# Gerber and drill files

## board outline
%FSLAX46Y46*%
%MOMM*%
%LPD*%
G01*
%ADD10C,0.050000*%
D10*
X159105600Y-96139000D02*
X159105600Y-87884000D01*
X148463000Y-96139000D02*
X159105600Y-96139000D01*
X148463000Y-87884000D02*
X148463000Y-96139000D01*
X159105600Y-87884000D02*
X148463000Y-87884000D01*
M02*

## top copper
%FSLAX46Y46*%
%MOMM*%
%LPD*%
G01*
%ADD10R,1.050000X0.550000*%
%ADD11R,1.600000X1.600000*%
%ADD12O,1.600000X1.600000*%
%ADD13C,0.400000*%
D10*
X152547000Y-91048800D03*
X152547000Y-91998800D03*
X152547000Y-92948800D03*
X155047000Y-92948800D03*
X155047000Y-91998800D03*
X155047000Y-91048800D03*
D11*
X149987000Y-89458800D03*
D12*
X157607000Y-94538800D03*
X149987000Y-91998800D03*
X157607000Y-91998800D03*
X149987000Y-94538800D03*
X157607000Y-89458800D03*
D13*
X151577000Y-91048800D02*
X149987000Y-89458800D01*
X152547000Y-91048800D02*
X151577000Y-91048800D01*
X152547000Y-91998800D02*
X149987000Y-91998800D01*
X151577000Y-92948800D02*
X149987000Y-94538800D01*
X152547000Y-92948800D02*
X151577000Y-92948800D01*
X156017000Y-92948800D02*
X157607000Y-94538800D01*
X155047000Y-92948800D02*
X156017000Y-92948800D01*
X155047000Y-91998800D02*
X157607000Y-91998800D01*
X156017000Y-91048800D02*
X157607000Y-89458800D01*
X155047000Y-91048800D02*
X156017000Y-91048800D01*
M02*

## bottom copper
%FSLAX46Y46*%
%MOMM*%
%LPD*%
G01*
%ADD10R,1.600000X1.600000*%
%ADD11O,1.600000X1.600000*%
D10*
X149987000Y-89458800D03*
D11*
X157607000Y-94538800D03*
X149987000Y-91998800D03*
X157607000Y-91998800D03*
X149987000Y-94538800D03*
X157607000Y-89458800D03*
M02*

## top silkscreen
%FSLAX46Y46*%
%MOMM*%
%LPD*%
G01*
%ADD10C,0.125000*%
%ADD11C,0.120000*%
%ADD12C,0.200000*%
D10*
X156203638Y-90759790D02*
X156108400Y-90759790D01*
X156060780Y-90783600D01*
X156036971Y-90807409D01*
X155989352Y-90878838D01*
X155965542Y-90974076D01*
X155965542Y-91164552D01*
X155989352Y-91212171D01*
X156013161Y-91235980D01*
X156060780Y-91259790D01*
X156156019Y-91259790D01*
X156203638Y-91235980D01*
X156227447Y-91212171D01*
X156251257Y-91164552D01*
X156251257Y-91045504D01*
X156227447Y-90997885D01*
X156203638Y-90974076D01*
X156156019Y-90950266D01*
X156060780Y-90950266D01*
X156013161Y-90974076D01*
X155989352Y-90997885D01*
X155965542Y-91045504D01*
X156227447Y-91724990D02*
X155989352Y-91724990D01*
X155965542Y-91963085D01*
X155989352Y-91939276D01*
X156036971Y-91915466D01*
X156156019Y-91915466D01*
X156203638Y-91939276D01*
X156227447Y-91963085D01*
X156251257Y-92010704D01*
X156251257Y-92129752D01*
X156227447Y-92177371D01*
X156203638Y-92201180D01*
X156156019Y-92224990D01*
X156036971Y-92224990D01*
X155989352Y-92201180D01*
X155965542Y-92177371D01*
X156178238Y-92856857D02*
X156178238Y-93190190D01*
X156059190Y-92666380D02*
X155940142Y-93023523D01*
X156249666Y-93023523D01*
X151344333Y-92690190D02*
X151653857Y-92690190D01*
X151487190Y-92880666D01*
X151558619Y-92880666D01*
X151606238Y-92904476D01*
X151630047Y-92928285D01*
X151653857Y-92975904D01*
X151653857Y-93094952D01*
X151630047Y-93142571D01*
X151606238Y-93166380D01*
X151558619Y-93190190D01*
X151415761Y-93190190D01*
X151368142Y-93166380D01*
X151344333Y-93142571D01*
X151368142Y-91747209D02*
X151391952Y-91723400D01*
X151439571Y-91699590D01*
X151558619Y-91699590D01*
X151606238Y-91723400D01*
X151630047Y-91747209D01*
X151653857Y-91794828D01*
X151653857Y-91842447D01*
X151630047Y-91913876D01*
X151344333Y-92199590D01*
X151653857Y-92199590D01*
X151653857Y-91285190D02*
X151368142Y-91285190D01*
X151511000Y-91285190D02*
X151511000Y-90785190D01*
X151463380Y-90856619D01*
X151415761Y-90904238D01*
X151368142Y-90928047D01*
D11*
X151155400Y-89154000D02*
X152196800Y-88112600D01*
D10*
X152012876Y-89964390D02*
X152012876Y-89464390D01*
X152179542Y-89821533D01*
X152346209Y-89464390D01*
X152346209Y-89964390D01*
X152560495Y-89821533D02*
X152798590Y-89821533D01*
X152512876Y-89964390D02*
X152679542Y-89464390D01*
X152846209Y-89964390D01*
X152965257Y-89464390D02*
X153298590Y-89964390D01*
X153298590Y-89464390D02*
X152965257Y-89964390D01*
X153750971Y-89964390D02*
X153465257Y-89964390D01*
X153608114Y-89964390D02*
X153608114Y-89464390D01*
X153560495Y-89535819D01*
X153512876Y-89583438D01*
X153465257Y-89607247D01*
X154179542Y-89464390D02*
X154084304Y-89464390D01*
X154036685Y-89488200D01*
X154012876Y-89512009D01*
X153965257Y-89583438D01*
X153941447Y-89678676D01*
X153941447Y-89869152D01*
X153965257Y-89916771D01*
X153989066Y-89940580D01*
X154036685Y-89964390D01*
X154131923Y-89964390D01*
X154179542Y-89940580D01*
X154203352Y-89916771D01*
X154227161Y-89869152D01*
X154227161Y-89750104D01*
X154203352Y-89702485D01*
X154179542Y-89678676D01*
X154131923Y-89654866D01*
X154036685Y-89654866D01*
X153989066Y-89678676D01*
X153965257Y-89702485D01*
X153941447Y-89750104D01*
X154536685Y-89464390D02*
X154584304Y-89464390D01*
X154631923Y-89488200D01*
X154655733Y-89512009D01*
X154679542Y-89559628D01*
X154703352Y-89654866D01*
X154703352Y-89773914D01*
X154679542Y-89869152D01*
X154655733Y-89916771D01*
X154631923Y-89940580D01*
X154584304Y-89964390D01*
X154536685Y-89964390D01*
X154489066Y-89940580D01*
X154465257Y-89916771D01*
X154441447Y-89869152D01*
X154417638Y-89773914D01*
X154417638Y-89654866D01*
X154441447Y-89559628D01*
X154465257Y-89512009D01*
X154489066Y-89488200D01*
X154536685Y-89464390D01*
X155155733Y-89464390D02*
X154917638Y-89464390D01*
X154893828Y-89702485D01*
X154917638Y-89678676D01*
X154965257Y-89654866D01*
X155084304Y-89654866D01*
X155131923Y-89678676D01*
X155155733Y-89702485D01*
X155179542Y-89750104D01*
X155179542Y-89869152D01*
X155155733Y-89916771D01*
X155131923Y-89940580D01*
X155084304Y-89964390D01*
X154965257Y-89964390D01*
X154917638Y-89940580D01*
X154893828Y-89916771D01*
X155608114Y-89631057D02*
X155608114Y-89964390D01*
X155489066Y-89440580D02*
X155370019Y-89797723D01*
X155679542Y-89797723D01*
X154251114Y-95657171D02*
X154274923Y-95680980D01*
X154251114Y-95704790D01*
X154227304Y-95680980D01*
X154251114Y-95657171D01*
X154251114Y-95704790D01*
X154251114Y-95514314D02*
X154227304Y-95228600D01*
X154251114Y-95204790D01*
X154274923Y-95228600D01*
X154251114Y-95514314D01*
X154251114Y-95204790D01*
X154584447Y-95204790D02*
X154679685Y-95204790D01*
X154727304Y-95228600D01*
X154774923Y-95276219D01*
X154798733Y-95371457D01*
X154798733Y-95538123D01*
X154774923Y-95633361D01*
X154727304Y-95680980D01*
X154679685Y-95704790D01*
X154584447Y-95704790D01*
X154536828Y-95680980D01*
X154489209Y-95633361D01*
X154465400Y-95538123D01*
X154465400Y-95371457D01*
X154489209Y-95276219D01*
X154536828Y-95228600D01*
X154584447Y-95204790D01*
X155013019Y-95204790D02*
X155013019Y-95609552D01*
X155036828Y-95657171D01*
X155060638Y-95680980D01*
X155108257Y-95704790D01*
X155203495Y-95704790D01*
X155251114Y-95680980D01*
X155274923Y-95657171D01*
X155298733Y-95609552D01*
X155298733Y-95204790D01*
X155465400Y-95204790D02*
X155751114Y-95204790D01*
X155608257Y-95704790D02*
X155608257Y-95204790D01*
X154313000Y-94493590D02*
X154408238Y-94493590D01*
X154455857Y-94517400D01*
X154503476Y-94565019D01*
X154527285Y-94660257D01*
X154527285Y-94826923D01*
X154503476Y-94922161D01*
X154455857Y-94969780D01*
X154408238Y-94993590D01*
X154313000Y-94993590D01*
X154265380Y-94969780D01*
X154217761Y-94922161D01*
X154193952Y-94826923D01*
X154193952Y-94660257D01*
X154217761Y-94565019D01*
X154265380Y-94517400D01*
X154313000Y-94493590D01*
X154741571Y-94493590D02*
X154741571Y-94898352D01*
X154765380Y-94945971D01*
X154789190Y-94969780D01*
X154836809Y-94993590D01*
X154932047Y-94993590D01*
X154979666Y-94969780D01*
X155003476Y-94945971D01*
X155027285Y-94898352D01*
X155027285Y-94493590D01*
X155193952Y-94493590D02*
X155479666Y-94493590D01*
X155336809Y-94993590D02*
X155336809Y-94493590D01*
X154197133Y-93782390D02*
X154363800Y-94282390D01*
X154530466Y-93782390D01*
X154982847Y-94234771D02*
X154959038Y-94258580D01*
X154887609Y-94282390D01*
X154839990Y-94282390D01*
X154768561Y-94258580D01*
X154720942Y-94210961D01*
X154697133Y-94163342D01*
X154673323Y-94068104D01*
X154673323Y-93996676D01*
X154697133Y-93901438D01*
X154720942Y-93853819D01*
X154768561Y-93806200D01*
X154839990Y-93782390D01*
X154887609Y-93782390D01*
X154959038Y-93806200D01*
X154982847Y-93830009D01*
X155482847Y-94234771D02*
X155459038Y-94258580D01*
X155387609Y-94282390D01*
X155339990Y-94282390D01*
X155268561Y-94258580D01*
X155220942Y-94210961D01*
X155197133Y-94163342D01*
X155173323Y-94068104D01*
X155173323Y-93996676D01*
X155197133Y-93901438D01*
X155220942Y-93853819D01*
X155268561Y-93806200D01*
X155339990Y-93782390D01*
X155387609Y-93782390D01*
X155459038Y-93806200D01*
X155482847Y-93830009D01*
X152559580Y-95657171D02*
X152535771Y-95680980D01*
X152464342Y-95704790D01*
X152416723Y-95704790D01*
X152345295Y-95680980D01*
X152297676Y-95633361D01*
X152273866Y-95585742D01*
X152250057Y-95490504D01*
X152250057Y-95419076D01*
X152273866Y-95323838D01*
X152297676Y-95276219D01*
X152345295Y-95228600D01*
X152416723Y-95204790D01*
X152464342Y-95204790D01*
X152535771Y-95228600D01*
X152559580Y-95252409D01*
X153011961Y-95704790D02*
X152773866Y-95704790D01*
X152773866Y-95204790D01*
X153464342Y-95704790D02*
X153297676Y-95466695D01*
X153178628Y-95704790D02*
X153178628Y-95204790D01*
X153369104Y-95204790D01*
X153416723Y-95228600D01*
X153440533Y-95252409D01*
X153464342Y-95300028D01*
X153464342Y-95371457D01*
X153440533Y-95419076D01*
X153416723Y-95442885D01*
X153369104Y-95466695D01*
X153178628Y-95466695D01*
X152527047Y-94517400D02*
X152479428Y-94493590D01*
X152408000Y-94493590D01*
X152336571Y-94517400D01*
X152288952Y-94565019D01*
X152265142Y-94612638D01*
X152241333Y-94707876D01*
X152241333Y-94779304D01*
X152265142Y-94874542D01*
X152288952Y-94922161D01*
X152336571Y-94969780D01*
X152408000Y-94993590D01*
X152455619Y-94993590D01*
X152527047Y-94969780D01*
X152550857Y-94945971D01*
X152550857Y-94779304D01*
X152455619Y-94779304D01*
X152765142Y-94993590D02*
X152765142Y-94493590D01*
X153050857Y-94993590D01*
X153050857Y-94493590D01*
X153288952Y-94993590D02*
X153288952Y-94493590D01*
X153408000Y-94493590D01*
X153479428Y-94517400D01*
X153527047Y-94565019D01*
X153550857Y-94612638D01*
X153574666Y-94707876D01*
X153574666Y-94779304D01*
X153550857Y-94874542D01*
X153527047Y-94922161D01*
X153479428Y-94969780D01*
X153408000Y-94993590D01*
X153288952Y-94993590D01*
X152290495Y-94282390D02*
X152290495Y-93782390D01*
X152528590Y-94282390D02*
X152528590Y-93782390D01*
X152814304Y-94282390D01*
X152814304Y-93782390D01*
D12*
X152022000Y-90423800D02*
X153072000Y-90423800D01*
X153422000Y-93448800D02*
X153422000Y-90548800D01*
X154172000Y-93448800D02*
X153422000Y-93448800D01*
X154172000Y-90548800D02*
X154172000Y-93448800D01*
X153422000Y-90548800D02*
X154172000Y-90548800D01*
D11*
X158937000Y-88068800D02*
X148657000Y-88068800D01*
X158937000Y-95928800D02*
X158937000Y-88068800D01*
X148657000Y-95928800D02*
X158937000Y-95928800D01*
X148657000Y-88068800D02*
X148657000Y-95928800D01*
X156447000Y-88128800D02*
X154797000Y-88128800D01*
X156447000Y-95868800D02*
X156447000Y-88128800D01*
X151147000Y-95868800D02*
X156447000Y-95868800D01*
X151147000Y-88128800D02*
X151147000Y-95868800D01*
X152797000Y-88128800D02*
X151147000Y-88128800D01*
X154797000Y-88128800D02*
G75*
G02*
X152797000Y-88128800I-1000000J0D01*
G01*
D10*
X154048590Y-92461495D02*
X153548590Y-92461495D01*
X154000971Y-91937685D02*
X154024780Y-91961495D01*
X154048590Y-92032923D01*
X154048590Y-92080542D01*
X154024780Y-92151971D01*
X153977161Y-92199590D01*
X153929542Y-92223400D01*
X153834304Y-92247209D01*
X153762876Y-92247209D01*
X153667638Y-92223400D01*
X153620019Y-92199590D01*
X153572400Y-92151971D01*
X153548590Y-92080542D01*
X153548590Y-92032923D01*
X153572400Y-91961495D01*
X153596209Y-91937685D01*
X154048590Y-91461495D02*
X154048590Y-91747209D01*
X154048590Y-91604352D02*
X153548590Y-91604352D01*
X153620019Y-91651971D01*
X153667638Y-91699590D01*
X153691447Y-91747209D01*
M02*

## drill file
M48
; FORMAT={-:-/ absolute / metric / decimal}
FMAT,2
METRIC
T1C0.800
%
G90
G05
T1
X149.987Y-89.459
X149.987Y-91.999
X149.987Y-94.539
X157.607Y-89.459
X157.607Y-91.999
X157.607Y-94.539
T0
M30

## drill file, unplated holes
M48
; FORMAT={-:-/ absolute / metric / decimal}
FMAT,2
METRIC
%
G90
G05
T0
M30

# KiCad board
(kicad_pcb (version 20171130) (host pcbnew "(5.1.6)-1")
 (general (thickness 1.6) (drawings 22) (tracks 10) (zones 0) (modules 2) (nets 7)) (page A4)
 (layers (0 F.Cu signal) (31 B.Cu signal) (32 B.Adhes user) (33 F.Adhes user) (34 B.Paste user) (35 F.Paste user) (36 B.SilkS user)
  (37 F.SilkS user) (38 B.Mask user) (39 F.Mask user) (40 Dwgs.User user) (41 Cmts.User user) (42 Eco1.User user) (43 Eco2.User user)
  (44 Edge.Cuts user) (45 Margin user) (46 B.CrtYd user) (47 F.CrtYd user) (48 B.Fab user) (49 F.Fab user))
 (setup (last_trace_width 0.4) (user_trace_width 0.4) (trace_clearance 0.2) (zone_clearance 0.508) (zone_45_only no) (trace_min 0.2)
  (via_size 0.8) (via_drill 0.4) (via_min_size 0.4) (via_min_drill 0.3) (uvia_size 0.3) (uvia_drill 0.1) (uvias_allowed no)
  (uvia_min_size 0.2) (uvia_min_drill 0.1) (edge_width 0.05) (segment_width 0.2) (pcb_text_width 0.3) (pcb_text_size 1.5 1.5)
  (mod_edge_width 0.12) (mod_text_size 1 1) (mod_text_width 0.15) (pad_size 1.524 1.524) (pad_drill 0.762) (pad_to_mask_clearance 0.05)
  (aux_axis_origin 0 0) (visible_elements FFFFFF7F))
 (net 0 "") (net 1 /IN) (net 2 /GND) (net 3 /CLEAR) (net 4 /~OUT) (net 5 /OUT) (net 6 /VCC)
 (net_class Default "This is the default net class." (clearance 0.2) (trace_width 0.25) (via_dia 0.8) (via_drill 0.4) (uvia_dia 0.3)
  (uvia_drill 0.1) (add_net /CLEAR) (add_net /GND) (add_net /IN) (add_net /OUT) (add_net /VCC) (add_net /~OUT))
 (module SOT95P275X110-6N (layer F.Cu) (at 153.797 91.9988)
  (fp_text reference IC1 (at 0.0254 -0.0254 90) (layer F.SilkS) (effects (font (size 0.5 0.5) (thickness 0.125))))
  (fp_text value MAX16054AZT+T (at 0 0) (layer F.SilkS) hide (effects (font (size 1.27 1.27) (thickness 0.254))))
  (fp_line (start -1.775 -1.575) (end -0.725 -1.575) (layer F.SilkS) (width 0.2))
  (fp_line (start -0.375 1.45) (end -0.375 -1.45) (layer F.SilkS) (width 0.2))
  (fp_line (start 0.375 1.45) (end -0.375 1.45) (layer F.SilkS) (width 0.2))
  (fp_line (start 0.375 -1.45) (end 0.375 1.45) (layer F.SilkS) (width 0.2))
  (fp_line (start -0.375 -1.45) (end 0.375 -1.45) (layer F.SilkS) (width 0.2))
  (pad 1 smd rect (at -1.25 -0.95 90) (size 0.55 1.05) (layers F.Cu F.Paste F.Mask) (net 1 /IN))
  (pad 2 smd rect (at -1.25 0 90) (size 0.55 1.05) (layers F.Cu F.Paste F.Mask) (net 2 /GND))
  (pad 3 smd rect (at -1.25 0.95 90) (size 0.55 1.05) (layers F.Cu F.Paste F.Mask) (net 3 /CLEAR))
  (pad 4 smd rect (at 1.25 0.95 90) (size 0.55 1.05) (layers F.Cu F.Paste F.Mask) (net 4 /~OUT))
  (pad 5 smd rect (at 1.25 0 90) (size 0.55 1.05) (layers F.Cu F.Paste F.Mask) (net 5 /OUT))
  (pad 6 smd rect (at 1.25 -0.95 90) (size 0.55 1.05) (layers F.Cu F.Paste F.Mask) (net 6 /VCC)))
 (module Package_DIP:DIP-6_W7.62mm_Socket (layer F.Cu) (at 149.987 89.4588)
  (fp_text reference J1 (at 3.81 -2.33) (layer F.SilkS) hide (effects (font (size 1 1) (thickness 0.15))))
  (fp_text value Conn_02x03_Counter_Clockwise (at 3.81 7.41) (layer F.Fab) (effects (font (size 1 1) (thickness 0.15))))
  (fp_line (start 8.95 -1.39) (end -1.33 -1.39) (layer F.SilkS) (width 0.12))
  (fp_line (start 8.95 6.47) (end 8.95 -1.39) (layer F.SilkS) (width 0.12))
  (fp_line (start -1.33 6.47) (end 8.95 6.47) (layer F.SilkS) (width 0.12))
  (fp_line (start -1.33 -1.39) (end -1.33 6.47) (layer F.SilkS) (width 0.12))
  (fp_line (start 6.46 -1.33) (end 4.81 -1.33) (layer F.SilkS) (width 0.12))
  (fp_line (start 6.46 6.41) (end 6.46 -1.33) (layer F.SilkS) (width 0.12))
  (fp_line (start 1.16 6.41) (end 6.46 6.41) (layer F.SilkS) (width 0.12))
  (fp_line (start 1.16 -1.33) (end 1.16 6.41) (layer F.SilkS) (width 0.12))
  (fp_line (start 2.81 -1.33) (end 1.16 -1.33) (layer F.SilkS) (width 0.12))
  (fp_arc (start 3.81 -1.33) (end 2.81 -1.33) (angle -180) (layer F.SilkS) (width 0.12))
  (pad 1 thru_hole rect (at 0 0) (size 1.6 1.6) (drill 0.8) (layers *.Cu *.Mask) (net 1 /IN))
  (pad 4 thru_hole oval (at 7.62 5.08) (size 1.6 1.6) (drill 0.8) (layers *.Cu *.Mask) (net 4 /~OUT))
  (pad 2 thru_hole oval (at 0 2.54) (size 1.6 1.6) (drill 0.8) (layers *.Cu *.Mask) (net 2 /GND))
  (pad 5 thru_hole oval (at 7.62 2.54) (size 1.6 1.6) (drill 0.8) (layers *.Cu *.Mask) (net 5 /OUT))
  (pad 3 thru_hole oval (at 0 5.08) (size 1.6 1.6) (drill 0.8) (layers *.Cu *.Mask) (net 3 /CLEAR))
  (pad 6 thru_hole oval (at 7.62 0) (size 1.6 1.6) (drill 0.8) (layers *.Cu *.Mask) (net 6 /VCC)))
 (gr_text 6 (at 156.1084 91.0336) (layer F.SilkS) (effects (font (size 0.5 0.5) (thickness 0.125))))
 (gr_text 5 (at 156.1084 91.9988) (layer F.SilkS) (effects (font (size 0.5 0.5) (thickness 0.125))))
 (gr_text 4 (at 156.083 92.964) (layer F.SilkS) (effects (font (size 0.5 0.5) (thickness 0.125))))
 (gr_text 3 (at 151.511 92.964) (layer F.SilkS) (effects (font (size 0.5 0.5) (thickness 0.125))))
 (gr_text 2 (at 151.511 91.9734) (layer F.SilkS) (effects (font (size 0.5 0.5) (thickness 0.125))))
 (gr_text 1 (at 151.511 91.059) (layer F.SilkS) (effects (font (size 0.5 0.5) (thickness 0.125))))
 (gr_line (start 151.1554 89.154) (end 152.1968 88.1126) (layer F.SilkS) (width 0.12))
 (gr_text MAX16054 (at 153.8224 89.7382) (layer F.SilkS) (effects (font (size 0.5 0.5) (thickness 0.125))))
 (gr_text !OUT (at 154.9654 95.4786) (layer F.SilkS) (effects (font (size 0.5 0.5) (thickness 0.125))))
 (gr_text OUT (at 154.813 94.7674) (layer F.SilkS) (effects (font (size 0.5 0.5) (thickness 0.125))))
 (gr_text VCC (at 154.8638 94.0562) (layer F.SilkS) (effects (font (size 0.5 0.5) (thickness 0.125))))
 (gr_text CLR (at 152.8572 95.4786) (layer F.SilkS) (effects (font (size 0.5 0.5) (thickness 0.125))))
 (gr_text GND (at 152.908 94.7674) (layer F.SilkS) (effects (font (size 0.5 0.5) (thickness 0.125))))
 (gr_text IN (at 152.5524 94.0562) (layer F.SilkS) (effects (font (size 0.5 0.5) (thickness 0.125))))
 (gr_line (start 159.1056 96.139) (end 159.1056 87.884) (layer Edge.Cuts) (width 0.05))
 (gr_line (start 148.463 96.139) (end 159.1056 96.139) (layer Edge.Cuts) (width 0.05))
 (gr_line (start 148.463 87.884) (end 148.463 96.139) (layer Edge.Cuts) (width 0.05))
 (gr_line (start 159.1056 87.884) (end 148.463 87.884) (layer Edge.Cuts) (width 0.05))
 (segment (start 151.577 91.0488) (end 149.987 89.4588) (width 0.4) (layer F.Cu) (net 1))
 (segment (start 152.547 91.0488) (end 151.577 91.0488) (width 0.4) (layer F.Cu) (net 1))
 (segment (start 152.547 91.9988) (end 149.987 91.9988) (width 0.4) (layer F.Cu) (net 2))
 (segment (start 151.577 92.9488) (end 149.987 94.5388) (width 0.4) (layer F.Cu) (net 3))
 (segment (start 152.547 92.9488) (end 151.577 92.9488) (width 0.4) (layer F.Cu) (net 3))
 (segment (start 156.017 92.9488) (end 157.607 94.5388) (width 0.4) (layer F.Cu) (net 4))
 (segment (start 155.047 92.9488) (end 156.017 92.9488) (width 0.4) (layer F.Cu) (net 4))
 (segment (start 155.047 91.9988) (end 157.607 91.9988) (width 0.4) (layer F.Cu) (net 5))
 (segment (start 156.017 91.0488) (end 157.607 89.4588) (width 0.4) (layer F.Cu) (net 6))
 (segment (start 155.047 91.0488) (end 156.017 91.0488) (width 0.4) (layer F.Cu) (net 6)))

